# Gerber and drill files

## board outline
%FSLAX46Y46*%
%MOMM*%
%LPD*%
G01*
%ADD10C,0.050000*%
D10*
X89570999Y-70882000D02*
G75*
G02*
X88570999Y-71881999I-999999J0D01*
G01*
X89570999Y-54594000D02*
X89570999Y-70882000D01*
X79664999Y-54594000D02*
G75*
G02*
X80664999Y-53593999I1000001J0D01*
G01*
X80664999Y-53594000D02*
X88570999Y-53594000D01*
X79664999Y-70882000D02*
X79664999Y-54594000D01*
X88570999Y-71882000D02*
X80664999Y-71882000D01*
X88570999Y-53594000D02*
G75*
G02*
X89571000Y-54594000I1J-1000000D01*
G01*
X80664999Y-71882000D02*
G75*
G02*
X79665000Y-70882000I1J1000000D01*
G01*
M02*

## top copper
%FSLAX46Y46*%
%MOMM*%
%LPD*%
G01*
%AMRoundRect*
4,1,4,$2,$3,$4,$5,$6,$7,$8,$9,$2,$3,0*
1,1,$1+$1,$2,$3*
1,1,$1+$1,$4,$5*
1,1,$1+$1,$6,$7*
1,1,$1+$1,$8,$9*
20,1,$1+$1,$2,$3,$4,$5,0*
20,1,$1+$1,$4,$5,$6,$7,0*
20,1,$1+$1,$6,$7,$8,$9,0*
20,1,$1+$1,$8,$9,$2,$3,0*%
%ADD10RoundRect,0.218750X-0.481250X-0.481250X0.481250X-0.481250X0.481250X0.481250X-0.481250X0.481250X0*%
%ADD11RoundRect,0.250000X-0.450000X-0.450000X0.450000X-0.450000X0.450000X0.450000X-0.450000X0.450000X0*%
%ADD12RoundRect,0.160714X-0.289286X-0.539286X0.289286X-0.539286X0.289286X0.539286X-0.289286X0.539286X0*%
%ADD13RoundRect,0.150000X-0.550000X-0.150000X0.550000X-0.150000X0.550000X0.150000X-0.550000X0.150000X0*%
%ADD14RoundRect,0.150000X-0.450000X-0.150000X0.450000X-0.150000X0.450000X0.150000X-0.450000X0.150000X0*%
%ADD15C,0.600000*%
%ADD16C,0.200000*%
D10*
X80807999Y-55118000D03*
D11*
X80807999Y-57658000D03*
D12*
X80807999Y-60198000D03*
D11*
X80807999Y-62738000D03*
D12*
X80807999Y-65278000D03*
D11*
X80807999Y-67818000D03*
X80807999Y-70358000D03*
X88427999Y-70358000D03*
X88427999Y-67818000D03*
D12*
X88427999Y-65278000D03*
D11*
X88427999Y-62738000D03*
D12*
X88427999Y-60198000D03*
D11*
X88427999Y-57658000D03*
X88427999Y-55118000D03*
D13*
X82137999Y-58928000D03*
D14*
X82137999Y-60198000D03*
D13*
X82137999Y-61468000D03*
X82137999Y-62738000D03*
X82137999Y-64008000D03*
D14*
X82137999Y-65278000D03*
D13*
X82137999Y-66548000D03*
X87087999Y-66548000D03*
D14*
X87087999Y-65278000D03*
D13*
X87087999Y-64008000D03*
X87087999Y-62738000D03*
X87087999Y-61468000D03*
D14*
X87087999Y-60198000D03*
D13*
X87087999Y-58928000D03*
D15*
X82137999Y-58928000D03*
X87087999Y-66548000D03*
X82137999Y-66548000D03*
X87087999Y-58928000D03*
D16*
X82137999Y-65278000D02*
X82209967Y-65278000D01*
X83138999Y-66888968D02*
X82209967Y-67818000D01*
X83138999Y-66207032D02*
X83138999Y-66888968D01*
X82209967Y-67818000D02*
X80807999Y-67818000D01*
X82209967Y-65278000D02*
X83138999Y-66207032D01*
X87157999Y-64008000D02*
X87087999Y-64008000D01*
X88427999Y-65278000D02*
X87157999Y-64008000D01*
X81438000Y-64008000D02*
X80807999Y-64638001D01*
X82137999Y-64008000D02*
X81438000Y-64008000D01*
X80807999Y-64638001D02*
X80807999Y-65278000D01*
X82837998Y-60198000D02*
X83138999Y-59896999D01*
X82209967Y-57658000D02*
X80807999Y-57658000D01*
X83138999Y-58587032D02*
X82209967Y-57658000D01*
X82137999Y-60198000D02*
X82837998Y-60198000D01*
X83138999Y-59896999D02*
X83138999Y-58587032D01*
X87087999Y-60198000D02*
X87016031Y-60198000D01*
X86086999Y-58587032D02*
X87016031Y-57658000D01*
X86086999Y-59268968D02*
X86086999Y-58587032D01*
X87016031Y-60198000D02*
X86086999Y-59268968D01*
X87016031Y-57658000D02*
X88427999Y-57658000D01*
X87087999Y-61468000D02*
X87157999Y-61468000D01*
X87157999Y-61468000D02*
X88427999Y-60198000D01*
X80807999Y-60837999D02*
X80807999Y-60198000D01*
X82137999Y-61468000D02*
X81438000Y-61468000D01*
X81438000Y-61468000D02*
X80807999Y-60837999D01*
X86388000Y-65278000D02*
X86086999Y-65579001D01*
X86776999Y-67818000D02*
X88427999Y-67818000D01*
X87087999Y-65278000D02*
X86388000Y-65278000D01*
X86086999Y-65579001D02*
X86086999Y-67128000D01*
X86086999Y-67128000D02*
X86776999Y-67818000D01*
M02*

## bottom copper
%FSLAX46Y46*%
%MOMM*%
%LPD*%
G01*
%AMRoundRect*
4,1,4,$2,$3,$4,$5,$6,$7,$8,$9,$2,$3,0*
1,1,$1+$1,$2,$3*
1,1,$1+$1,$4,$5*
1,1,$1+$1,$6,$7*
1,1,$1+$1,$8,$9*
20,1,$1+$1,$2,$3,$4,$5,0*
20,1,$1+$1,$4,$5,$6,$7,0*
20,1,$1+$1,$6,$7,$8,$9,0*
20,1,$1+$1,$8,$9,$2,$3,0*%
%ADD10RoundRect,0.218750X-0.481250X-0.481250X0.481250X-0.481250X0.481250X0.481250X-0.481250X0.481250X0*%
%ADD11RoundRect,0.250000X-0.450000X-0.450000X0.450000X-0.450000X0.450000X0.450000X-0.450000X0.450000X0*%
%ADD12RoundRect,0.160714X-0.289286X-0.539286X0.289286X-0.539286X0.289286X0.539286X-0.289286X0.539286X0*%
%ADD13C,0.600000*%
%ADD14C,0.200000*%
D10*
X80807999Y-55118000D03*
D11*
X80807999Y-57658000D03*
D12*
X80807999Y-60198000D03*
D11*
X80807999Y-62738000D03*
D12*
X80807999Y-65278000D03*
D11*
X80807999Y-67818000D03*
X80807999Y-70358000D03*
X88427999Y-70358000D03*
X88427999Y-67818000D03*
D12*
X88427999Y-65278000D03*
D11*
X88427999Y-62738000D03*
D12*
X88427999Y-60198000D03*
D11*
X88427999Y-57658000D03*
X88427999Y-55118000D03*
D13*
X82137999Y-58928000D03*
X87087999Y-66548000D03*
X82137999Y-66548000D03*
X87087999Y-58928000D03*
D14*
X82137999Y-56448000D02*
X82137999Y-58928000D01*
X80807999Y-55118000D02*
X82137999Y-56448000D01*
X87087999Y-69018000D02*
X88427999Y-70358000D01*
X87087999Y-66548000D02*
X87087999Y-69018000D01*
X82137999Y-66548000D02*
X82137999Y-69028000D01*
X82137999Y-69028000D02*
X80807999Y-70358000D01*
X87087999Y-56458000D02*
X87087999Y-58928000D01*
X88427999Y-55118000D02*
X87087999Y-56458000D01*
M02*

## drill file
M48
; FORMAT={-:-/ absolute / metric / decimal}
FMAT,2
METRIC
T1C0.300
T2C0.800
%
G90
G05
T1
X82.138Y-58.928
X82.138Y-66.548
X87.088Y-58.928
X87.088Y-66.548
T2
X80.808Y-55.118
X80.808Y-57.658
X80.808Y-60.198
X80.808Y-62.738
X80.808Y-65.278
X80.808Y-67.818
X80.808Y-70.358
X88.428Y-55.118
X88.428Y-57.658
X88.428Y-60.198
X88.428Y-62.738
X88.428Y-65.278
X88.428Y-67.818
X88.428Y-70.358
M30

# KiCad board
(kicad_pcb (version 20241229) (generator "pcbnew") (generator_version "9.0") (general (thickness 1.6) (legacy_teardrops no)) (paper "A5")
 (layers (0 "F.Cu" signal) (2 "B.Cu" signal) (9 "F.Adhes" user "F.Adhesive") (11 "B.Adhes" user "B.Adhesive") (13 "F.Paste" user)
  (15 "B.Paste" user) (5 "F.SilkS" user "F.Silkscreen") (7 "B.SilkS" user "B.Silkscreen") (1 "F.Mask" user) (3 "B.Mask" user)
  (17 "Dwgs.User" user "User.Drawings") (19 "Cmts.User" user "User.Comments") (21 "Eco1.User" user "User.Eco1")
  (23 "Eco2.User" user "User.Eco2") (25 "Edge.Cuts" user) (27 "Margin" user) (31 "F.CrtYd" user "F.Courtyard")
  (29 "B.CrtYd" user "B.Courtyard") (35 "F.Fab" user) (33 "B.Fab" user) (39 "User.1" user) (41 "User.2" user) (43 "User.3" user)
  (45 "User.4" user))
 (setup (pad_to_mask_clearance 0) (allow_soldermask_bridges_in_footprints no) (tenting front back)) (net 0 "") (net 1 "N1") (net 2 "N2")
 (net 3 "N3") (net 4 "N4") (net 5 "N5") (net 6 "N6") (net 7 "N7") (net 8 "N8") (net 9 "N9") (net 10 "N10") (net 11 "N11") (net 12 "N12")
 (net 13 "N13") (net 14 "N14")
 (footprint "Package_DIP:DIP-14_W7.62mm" (layer "F.Cu") (at 80.807999 55.118)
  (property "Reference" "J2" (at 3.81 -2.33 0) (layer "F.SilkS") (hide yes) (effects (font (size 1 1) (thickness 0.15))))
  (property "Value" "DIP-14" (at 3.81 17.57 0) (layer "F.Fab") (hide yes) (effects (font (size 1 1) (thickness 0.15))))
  (pad "1" thru_hole roundrect (at 0 0) (size 1.4 1.4) (drill 0.8) (layers "*.Cu" "*.Mask") (remove_unused_layers no)
   (roundrect_rratio 0.15625) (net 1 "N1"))
  (pad "2" thru_hole roundrect (at 0 2.54) (size 1.4 1.4) (drill 0.8) (layers "*.Cu" "*.Mask") (remove_unused_layers no)
   (roundrect_rratio 0.1785714286) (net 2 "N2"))
  (pad "3" thru_hole roundrect (at 0 5.08) (size 0.9 1.4) (drill 0.8) (layers "*.Cu" "*.Mask") (remove_unused_layers no)
   (roundrect_rratio 0.1785714286) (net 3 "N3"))
  (pad "4" thru_hole roundrect (at 0 7.62) (size 1.4 1.4) (drill 0.8) (layers "*.Cu" "*.Mask") (remove_unused_layers no)
   (roundrect_rratio 0.1785714286) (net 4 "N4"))
  (pad "5" thru_hole roundrect (at 0 10.16) (size 0.9 1.4) (drill 0.8) (layers "*.Cu" "*.Mask") (remove_unused_layers no)
   (roundrect_rratio 0.1785714286) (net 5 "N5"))
  (pad "6" thru_hole roundrect (at 0 12.7) (size 1.4 1.4) (drill 0.8) (layers "*.Cu" "*.Mask") (remove_unused_layers no)
   (roundrect_rratio 0.1785714286) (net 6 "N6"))
  (pad "7" thru_hole roundrect (at 0 15.24) (size 1.4 1.4) (drill 0.8) (layers "*.Cu" "*.Mask") (remove_unused_layers no)
   (roundrect_rratio 0.1785714286) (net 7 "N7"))
  (pad "8" thru_hole roundrect (at 7.62 15.24) (size 1.4 1.4) (drill 0.8) (layers "*.Cu" "*.Mask") (remove_unused_layers no)
   (roundrect_rratio 0.1785714286) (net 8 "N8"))
  (pad "9" thru_hole roundrect (at 7.62 12.7) (size 1.4 1.4) (drill 0.8) (layers "*.Cu" "*.Mask") (remove_unused_layers no)
   (roundrect_rratio 0.1785714286) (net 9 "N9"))
  (pad "10" thru_hole roundrect (at 7.62 10.16) (size 0.9 1.4) (drill 0.8) (layers "*.Cu" "*.Mask") (remove_unused_layers no)
   (roundrect_rratio 0.1785714286) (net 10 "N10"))
  (pad "11" thru_hole roundrect (at 7.62 7.62) (size 1.4 1.4) (drill 0.8) (layers "*.Cu" "*.Mask") (remove_unused_layers no)
   (roundrect_rratio 0.1785714286) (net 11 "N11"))
  (pad "12" thru_hole roundrect (at 7.62 5.08) (size 0.9 1.4) (drill 0.8) (layers "*.Cu" "*.Mask") (remove_unused_layers no)
   (roundrect_rratio 0.1785714286) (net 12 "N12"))
  (pad "13" thru_hole roundrect (at 7.62 2.54) (size 1.4 1.4) (drill 0.8) (layers "*.Cu" "*.Mask") (remove_unused_layers no)
   (roundrect_rratio 0.1785714286) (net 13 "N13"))
  (pad "14" thru_hole roundrect (at 7.62 0) (size 1.4 1.4) (drill 0.8) (layers "*.Cu" "*.Mask") (remove_unused_layers no)
   (roundrect_rratio 0.1785714286) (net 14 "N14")))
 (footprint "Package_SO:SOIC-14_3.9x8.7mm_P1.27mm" (layer "F.Cu") (at 84.612999 62.738)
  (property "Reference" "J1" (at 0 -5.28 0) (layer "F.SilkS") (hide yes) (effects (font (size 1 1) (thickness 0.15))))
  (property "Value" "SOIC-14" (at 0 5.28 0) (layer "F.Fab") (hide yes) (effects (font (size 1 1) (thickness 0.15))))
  (pad "1" smd roundrect (at -2.475 -3.81) (size 1.4 0.6) (layers "F.Cu" "F.Mask" "F.Paste") (roundrect_rratio 0.25) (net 1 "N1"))
  (pad "2" smd roundrect (at -2.475 -2.54) (size 1.2 0.6) (layers "F.Cu" "F.Mask" "F.Paste") (roundrect_rratio 0.25) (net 2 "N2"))
  (pad "3" smd roundrect (at -2.475 -1.27) (size 1.4 0.6) (layers "F.Cu" "F.Mask" "F.Paste") (roundrect_rratio 0.25) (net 3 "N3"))
  (pad "4" smd roundrect (at -2.475 0) (size 1.4 0.6) (layers "F.Cu" "F.Mask" "F.Paste") (roundrect_rratio 0.25) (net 4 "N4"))
  (pad "5" smd roundrect (at -2.475 1.27) (size 1.4 0.6) (layers "F.Cu" "F.Mask" "F.Paste") (roundrect_rratio 0.25) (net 5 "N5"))
  (pad "6" smd roundrect (at -2.475 2.54) (size 1.2 0.6) (layers "F.Cu" "F.Mask" "F.Paste") (roundrect_rratio 0.25) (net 6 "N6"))
  (pad "7" smd roundrect (at -2.475 3.81) (size 1.4 0.6) (layers "F.Cu" "F.Mask" "F.Paste") (roundrect_rratio 0.25) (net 7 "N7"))
  (pad "8" smd roundrect (at 2.475 3.81) (size 1.4 0.6) (layers "F.Cu" "F.Mask" "F.Paste") (roundrect_rratio 0.25) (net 8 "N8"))
  (pad "9" smd roundrect (at 2.475 2.54) (size 1.2 0.6) (layers "F.Cu" "F.Mask" "F.Paste") (roundrect_rratio 0.25) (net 9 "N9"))
  (pad "10" smd roundrect (at 2.475 1.27) (size 1.4 0.6) (layers "F.Cu" "F.Mask" "F.Paste") (roundrect_rratio 0.25) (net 10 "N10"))
  (pad "11" smd roundrect (at 2.475 0) (size 1.4 0.6) (layers "F.Cu" "F.Mask" "F.Paste") (roundrect_rratio 0.25) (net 11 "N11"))
  (pad "12" smd roundrect (at 2.475 -1.27) (size 1.4 0.6) (layers "F.Cu" "F.Mask" "F.Paste") (roundrect_rratio 0.25) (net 12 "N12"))
  (pad "13" smd roundrect (at 2.475 -2.54) (size 1.2 0.6) (layers "F.Cu" "F.Mask" "F.Paste") (roundrect_rratio 0.25) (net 13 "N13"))
  (pad "14" smd roundrect (at 2.475 -3.81) (size 1.4 0.6) (layers "F.Cu" "F.Mask" "F.Paste") (roundrect_rratio 0.25) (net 14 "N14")))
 (gr_arc (start 89.570999 70.882) (mid 89.278106 71.589107) (end 88.570999 71.882) (stroke (width 0.05) (type default)) (layer "Edge.Cuts"))
 (gr_line (start 89.570999 54.594) (end 89.570999 70.882) (stroke (width 0.05) (type default)) (layer "Edge.Cuts"))
 (gr_arc (start 79.664999 54.594) (mid 79.957892 53.886893) (end 80.664999 53.594) (stroke (width 0.05) (type default)) (layer "Edge.Cuts"))
 (gr_line (start 80.664999 53.594) (end 88.570999 53.594) (stroke (width 0.05) (type default)) (layer "Edge.Cuts"))
 (gr_line (start 79.664999 70.882) (end 79.664999 54.594) (stroke (width 0.05) (type default)) (layer "Edge.Cuts"))
 (gr_line (start 88.570999 71.882) (end 80.664999 71.882) (stroke (width 0.05) (type default)) (layer "Edge.Cuts"))
 (gr_arc (start 88.570999 53.594) (mid 89.278106 53.886893) (end 89.570999 54.594) (stroke (width 0.05) (type default)) (layer "Edge.Cuts"))
 (gr_arc (start 80.664999 71.882) (mid 79.957892 71.589107) (end 79.664999 70.882) (stroke (width 0.05) (type default)) (layer "Edge.Cuts"))
 (segment (start 82.137999 65.278) (end 82.209967 65.278) (width 0.2) (layer "F.Cu") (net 6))
 (segment (start 83.138999 66.888968) (end 82.209967 67.818) (width 0.2) (layer "F.Cu") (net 6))
 (segment (start 83.138999 66.207032) (end 83.138999 66.888968) (width 0.2) (layer "F.Cu") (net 6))
 (segment (start 82.209967 67.818) (end 80.807999 67.818) (width 0.2) (layer "F.Cu") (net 6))
 (segment (start 82.209967 65.278) (end 83.138999 66.207032) (width 0.2) (layer "F.Cu") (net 6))
 (segment (start 87.157999 64.008) (end 87.087999 64.008) (width 0.2) (layer "F.Cu") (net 10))
 (segment (start 88.427999 65.278) (end 87.157999 64.008) (width 0.2) (layer "F.Cu") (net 10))
 (via (at 82.137999 58.928) (size 0.6) (drill 0.3) (layers "F.Cu" "B.Cu") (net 1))
 (segment (start 82.137999 56.448) (end 82.137999 58.928) (width 0.2) (layer "B.Cu") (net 1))
 (segment (start 80.807999 55.118) (end 82.137999 56.448) (width 0.2) (layer "B.Cu") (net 1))
 (segment (start 81.438 64.008) (end 80.807999 64.638001) (width 0.2) (layer "F.Cu") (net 5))
 (segment (start 82.137999 64.008) (end 81.438 64.008) (width 0.2) (layer "F.Cu") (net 5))
 (segment (start 80.807999 64.638001) (end 80.807999 65.278) (width 0.2) (layer "F.Cu") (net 5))
 (segment (start 82.837998 60.198) (end 83.138999 59.896999) (width 0.2) (layer "F.Cu") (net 2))
 (segment (start 82.209967 57.658) (end 80.807999 57.658) (width 0.2) (layer "F.Cu") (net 2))
 (segment (start 83.138999 58.587032) (end 82.209967 57.658) (width 0.2) (layer "F.Cu") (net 2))
 (segment (start 82.137999 60.198) (end 82.837998 60.198) (width 0.2) (layer "F.Cu") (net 2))
 (segment (start 83.138999 59.896999) (end 83.138999 58.587032) (width 0.2) (layer "F.Cu") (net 2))
 (segment (start 87.087999 60.198) (end 87.016031 60.198) (width 0.2) (layer "F.Cu") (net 13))
 (segment (start 86.086999 58.587032) (end 87.016031 57.658) (width 0.2) (layer "F.Cu") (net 13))
 (segment (start 86.086999 59.268968) (end 86.086999 58.587032) (width 0.2) (layer "F.Cu") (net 13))
 (segment (start 87.016031 60.198) (end 86.086999 59.268968) (width 0.2) (layer "F.Cu") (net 13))
 (segment (start 87.016031 57.658) (end 88.427999 57.658) (width 0.2) (layer "F.Cu") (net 13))
 (segment (start 87.087999 61.468) (end 87.157999 61.468) (width 0.2) (layer "F.Cu") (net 12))
 (segment (start 87.157999 61.468) (end 88.427999 60.198) (width 0.2) (layer "F.Cu") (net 12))
 (via (at 87.087999 66.548) (size 0.6) (drill 0.3) (layers "F.Cu" "B.Cu") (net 8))
 (segment (start 87.087999 69.018) (end 88.427999 70.358) (width 0.2) (layer "B.Cu") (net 8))
 (segment (start 87.087999 66.548) (end 87.087999 69.018) (width 0.2) (layer "B.Cu") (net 8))
 (via (at 82.137999 66.548) (size 0.6) (drill 0.3) (layers "F.Cu" "B.Cu") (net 7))
 (segment (start 82.137999 66.548) (end 82.137999 69.028) (width 0.2) (layer "B.Cu") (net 7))
 (segment (start 82.137999 69.028) (end 80.807999 70.358) (width 0.2) (layer "B.Cu") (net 7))
 (segment (start 80.807999 60.837999) (end 80.807999 60.198) (width 0.2) (layer "F.Cu") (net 3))
 (segment (start 82.137999 61.468) (end 81.438 61.468) (width 0.2) (layer "F.Cu") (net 3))
 (segment (start 81.438 61.468) (end 80.807999 60.837999) (width 0.2) (layer "F.Cu") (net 3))
 (via (at 87.087999 58.928) (size 0.6) (drill 0.3) (layers "F.Cu" "B.Cu") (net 14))
 (segment (start 87.087999 56.458) (end 87.087999 58.928) (width 0.2) (layer "B.Cu") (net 14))
 (segment (start 88.427999 55.118) (end 87.087999 56.458) (width 0.2) (layer "B.Cu") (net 14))
 (segment (start 86.388 65.278) (end 86.086999 65.579001) (width 0.2) (layer "F.Cu") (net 9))
 (segment (start 86.776999 67.818) (end 88.427999 67.818) (width 0.2) (layer "F.Cu") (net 9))
 (segment (start 87.087999 65.278) (end 86.388 65.278) (width 0.2) (layer "F.Cu") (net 9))
 (segment (start 86.086999 65.579001) (end 86.086999 67.128) (width 0.2) (layer "F.Cu") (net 9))
 (segment (start 86.086999 67.128) (end 86.776999 67.818) (width 0.2) (layer "F.Cu") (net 9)))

